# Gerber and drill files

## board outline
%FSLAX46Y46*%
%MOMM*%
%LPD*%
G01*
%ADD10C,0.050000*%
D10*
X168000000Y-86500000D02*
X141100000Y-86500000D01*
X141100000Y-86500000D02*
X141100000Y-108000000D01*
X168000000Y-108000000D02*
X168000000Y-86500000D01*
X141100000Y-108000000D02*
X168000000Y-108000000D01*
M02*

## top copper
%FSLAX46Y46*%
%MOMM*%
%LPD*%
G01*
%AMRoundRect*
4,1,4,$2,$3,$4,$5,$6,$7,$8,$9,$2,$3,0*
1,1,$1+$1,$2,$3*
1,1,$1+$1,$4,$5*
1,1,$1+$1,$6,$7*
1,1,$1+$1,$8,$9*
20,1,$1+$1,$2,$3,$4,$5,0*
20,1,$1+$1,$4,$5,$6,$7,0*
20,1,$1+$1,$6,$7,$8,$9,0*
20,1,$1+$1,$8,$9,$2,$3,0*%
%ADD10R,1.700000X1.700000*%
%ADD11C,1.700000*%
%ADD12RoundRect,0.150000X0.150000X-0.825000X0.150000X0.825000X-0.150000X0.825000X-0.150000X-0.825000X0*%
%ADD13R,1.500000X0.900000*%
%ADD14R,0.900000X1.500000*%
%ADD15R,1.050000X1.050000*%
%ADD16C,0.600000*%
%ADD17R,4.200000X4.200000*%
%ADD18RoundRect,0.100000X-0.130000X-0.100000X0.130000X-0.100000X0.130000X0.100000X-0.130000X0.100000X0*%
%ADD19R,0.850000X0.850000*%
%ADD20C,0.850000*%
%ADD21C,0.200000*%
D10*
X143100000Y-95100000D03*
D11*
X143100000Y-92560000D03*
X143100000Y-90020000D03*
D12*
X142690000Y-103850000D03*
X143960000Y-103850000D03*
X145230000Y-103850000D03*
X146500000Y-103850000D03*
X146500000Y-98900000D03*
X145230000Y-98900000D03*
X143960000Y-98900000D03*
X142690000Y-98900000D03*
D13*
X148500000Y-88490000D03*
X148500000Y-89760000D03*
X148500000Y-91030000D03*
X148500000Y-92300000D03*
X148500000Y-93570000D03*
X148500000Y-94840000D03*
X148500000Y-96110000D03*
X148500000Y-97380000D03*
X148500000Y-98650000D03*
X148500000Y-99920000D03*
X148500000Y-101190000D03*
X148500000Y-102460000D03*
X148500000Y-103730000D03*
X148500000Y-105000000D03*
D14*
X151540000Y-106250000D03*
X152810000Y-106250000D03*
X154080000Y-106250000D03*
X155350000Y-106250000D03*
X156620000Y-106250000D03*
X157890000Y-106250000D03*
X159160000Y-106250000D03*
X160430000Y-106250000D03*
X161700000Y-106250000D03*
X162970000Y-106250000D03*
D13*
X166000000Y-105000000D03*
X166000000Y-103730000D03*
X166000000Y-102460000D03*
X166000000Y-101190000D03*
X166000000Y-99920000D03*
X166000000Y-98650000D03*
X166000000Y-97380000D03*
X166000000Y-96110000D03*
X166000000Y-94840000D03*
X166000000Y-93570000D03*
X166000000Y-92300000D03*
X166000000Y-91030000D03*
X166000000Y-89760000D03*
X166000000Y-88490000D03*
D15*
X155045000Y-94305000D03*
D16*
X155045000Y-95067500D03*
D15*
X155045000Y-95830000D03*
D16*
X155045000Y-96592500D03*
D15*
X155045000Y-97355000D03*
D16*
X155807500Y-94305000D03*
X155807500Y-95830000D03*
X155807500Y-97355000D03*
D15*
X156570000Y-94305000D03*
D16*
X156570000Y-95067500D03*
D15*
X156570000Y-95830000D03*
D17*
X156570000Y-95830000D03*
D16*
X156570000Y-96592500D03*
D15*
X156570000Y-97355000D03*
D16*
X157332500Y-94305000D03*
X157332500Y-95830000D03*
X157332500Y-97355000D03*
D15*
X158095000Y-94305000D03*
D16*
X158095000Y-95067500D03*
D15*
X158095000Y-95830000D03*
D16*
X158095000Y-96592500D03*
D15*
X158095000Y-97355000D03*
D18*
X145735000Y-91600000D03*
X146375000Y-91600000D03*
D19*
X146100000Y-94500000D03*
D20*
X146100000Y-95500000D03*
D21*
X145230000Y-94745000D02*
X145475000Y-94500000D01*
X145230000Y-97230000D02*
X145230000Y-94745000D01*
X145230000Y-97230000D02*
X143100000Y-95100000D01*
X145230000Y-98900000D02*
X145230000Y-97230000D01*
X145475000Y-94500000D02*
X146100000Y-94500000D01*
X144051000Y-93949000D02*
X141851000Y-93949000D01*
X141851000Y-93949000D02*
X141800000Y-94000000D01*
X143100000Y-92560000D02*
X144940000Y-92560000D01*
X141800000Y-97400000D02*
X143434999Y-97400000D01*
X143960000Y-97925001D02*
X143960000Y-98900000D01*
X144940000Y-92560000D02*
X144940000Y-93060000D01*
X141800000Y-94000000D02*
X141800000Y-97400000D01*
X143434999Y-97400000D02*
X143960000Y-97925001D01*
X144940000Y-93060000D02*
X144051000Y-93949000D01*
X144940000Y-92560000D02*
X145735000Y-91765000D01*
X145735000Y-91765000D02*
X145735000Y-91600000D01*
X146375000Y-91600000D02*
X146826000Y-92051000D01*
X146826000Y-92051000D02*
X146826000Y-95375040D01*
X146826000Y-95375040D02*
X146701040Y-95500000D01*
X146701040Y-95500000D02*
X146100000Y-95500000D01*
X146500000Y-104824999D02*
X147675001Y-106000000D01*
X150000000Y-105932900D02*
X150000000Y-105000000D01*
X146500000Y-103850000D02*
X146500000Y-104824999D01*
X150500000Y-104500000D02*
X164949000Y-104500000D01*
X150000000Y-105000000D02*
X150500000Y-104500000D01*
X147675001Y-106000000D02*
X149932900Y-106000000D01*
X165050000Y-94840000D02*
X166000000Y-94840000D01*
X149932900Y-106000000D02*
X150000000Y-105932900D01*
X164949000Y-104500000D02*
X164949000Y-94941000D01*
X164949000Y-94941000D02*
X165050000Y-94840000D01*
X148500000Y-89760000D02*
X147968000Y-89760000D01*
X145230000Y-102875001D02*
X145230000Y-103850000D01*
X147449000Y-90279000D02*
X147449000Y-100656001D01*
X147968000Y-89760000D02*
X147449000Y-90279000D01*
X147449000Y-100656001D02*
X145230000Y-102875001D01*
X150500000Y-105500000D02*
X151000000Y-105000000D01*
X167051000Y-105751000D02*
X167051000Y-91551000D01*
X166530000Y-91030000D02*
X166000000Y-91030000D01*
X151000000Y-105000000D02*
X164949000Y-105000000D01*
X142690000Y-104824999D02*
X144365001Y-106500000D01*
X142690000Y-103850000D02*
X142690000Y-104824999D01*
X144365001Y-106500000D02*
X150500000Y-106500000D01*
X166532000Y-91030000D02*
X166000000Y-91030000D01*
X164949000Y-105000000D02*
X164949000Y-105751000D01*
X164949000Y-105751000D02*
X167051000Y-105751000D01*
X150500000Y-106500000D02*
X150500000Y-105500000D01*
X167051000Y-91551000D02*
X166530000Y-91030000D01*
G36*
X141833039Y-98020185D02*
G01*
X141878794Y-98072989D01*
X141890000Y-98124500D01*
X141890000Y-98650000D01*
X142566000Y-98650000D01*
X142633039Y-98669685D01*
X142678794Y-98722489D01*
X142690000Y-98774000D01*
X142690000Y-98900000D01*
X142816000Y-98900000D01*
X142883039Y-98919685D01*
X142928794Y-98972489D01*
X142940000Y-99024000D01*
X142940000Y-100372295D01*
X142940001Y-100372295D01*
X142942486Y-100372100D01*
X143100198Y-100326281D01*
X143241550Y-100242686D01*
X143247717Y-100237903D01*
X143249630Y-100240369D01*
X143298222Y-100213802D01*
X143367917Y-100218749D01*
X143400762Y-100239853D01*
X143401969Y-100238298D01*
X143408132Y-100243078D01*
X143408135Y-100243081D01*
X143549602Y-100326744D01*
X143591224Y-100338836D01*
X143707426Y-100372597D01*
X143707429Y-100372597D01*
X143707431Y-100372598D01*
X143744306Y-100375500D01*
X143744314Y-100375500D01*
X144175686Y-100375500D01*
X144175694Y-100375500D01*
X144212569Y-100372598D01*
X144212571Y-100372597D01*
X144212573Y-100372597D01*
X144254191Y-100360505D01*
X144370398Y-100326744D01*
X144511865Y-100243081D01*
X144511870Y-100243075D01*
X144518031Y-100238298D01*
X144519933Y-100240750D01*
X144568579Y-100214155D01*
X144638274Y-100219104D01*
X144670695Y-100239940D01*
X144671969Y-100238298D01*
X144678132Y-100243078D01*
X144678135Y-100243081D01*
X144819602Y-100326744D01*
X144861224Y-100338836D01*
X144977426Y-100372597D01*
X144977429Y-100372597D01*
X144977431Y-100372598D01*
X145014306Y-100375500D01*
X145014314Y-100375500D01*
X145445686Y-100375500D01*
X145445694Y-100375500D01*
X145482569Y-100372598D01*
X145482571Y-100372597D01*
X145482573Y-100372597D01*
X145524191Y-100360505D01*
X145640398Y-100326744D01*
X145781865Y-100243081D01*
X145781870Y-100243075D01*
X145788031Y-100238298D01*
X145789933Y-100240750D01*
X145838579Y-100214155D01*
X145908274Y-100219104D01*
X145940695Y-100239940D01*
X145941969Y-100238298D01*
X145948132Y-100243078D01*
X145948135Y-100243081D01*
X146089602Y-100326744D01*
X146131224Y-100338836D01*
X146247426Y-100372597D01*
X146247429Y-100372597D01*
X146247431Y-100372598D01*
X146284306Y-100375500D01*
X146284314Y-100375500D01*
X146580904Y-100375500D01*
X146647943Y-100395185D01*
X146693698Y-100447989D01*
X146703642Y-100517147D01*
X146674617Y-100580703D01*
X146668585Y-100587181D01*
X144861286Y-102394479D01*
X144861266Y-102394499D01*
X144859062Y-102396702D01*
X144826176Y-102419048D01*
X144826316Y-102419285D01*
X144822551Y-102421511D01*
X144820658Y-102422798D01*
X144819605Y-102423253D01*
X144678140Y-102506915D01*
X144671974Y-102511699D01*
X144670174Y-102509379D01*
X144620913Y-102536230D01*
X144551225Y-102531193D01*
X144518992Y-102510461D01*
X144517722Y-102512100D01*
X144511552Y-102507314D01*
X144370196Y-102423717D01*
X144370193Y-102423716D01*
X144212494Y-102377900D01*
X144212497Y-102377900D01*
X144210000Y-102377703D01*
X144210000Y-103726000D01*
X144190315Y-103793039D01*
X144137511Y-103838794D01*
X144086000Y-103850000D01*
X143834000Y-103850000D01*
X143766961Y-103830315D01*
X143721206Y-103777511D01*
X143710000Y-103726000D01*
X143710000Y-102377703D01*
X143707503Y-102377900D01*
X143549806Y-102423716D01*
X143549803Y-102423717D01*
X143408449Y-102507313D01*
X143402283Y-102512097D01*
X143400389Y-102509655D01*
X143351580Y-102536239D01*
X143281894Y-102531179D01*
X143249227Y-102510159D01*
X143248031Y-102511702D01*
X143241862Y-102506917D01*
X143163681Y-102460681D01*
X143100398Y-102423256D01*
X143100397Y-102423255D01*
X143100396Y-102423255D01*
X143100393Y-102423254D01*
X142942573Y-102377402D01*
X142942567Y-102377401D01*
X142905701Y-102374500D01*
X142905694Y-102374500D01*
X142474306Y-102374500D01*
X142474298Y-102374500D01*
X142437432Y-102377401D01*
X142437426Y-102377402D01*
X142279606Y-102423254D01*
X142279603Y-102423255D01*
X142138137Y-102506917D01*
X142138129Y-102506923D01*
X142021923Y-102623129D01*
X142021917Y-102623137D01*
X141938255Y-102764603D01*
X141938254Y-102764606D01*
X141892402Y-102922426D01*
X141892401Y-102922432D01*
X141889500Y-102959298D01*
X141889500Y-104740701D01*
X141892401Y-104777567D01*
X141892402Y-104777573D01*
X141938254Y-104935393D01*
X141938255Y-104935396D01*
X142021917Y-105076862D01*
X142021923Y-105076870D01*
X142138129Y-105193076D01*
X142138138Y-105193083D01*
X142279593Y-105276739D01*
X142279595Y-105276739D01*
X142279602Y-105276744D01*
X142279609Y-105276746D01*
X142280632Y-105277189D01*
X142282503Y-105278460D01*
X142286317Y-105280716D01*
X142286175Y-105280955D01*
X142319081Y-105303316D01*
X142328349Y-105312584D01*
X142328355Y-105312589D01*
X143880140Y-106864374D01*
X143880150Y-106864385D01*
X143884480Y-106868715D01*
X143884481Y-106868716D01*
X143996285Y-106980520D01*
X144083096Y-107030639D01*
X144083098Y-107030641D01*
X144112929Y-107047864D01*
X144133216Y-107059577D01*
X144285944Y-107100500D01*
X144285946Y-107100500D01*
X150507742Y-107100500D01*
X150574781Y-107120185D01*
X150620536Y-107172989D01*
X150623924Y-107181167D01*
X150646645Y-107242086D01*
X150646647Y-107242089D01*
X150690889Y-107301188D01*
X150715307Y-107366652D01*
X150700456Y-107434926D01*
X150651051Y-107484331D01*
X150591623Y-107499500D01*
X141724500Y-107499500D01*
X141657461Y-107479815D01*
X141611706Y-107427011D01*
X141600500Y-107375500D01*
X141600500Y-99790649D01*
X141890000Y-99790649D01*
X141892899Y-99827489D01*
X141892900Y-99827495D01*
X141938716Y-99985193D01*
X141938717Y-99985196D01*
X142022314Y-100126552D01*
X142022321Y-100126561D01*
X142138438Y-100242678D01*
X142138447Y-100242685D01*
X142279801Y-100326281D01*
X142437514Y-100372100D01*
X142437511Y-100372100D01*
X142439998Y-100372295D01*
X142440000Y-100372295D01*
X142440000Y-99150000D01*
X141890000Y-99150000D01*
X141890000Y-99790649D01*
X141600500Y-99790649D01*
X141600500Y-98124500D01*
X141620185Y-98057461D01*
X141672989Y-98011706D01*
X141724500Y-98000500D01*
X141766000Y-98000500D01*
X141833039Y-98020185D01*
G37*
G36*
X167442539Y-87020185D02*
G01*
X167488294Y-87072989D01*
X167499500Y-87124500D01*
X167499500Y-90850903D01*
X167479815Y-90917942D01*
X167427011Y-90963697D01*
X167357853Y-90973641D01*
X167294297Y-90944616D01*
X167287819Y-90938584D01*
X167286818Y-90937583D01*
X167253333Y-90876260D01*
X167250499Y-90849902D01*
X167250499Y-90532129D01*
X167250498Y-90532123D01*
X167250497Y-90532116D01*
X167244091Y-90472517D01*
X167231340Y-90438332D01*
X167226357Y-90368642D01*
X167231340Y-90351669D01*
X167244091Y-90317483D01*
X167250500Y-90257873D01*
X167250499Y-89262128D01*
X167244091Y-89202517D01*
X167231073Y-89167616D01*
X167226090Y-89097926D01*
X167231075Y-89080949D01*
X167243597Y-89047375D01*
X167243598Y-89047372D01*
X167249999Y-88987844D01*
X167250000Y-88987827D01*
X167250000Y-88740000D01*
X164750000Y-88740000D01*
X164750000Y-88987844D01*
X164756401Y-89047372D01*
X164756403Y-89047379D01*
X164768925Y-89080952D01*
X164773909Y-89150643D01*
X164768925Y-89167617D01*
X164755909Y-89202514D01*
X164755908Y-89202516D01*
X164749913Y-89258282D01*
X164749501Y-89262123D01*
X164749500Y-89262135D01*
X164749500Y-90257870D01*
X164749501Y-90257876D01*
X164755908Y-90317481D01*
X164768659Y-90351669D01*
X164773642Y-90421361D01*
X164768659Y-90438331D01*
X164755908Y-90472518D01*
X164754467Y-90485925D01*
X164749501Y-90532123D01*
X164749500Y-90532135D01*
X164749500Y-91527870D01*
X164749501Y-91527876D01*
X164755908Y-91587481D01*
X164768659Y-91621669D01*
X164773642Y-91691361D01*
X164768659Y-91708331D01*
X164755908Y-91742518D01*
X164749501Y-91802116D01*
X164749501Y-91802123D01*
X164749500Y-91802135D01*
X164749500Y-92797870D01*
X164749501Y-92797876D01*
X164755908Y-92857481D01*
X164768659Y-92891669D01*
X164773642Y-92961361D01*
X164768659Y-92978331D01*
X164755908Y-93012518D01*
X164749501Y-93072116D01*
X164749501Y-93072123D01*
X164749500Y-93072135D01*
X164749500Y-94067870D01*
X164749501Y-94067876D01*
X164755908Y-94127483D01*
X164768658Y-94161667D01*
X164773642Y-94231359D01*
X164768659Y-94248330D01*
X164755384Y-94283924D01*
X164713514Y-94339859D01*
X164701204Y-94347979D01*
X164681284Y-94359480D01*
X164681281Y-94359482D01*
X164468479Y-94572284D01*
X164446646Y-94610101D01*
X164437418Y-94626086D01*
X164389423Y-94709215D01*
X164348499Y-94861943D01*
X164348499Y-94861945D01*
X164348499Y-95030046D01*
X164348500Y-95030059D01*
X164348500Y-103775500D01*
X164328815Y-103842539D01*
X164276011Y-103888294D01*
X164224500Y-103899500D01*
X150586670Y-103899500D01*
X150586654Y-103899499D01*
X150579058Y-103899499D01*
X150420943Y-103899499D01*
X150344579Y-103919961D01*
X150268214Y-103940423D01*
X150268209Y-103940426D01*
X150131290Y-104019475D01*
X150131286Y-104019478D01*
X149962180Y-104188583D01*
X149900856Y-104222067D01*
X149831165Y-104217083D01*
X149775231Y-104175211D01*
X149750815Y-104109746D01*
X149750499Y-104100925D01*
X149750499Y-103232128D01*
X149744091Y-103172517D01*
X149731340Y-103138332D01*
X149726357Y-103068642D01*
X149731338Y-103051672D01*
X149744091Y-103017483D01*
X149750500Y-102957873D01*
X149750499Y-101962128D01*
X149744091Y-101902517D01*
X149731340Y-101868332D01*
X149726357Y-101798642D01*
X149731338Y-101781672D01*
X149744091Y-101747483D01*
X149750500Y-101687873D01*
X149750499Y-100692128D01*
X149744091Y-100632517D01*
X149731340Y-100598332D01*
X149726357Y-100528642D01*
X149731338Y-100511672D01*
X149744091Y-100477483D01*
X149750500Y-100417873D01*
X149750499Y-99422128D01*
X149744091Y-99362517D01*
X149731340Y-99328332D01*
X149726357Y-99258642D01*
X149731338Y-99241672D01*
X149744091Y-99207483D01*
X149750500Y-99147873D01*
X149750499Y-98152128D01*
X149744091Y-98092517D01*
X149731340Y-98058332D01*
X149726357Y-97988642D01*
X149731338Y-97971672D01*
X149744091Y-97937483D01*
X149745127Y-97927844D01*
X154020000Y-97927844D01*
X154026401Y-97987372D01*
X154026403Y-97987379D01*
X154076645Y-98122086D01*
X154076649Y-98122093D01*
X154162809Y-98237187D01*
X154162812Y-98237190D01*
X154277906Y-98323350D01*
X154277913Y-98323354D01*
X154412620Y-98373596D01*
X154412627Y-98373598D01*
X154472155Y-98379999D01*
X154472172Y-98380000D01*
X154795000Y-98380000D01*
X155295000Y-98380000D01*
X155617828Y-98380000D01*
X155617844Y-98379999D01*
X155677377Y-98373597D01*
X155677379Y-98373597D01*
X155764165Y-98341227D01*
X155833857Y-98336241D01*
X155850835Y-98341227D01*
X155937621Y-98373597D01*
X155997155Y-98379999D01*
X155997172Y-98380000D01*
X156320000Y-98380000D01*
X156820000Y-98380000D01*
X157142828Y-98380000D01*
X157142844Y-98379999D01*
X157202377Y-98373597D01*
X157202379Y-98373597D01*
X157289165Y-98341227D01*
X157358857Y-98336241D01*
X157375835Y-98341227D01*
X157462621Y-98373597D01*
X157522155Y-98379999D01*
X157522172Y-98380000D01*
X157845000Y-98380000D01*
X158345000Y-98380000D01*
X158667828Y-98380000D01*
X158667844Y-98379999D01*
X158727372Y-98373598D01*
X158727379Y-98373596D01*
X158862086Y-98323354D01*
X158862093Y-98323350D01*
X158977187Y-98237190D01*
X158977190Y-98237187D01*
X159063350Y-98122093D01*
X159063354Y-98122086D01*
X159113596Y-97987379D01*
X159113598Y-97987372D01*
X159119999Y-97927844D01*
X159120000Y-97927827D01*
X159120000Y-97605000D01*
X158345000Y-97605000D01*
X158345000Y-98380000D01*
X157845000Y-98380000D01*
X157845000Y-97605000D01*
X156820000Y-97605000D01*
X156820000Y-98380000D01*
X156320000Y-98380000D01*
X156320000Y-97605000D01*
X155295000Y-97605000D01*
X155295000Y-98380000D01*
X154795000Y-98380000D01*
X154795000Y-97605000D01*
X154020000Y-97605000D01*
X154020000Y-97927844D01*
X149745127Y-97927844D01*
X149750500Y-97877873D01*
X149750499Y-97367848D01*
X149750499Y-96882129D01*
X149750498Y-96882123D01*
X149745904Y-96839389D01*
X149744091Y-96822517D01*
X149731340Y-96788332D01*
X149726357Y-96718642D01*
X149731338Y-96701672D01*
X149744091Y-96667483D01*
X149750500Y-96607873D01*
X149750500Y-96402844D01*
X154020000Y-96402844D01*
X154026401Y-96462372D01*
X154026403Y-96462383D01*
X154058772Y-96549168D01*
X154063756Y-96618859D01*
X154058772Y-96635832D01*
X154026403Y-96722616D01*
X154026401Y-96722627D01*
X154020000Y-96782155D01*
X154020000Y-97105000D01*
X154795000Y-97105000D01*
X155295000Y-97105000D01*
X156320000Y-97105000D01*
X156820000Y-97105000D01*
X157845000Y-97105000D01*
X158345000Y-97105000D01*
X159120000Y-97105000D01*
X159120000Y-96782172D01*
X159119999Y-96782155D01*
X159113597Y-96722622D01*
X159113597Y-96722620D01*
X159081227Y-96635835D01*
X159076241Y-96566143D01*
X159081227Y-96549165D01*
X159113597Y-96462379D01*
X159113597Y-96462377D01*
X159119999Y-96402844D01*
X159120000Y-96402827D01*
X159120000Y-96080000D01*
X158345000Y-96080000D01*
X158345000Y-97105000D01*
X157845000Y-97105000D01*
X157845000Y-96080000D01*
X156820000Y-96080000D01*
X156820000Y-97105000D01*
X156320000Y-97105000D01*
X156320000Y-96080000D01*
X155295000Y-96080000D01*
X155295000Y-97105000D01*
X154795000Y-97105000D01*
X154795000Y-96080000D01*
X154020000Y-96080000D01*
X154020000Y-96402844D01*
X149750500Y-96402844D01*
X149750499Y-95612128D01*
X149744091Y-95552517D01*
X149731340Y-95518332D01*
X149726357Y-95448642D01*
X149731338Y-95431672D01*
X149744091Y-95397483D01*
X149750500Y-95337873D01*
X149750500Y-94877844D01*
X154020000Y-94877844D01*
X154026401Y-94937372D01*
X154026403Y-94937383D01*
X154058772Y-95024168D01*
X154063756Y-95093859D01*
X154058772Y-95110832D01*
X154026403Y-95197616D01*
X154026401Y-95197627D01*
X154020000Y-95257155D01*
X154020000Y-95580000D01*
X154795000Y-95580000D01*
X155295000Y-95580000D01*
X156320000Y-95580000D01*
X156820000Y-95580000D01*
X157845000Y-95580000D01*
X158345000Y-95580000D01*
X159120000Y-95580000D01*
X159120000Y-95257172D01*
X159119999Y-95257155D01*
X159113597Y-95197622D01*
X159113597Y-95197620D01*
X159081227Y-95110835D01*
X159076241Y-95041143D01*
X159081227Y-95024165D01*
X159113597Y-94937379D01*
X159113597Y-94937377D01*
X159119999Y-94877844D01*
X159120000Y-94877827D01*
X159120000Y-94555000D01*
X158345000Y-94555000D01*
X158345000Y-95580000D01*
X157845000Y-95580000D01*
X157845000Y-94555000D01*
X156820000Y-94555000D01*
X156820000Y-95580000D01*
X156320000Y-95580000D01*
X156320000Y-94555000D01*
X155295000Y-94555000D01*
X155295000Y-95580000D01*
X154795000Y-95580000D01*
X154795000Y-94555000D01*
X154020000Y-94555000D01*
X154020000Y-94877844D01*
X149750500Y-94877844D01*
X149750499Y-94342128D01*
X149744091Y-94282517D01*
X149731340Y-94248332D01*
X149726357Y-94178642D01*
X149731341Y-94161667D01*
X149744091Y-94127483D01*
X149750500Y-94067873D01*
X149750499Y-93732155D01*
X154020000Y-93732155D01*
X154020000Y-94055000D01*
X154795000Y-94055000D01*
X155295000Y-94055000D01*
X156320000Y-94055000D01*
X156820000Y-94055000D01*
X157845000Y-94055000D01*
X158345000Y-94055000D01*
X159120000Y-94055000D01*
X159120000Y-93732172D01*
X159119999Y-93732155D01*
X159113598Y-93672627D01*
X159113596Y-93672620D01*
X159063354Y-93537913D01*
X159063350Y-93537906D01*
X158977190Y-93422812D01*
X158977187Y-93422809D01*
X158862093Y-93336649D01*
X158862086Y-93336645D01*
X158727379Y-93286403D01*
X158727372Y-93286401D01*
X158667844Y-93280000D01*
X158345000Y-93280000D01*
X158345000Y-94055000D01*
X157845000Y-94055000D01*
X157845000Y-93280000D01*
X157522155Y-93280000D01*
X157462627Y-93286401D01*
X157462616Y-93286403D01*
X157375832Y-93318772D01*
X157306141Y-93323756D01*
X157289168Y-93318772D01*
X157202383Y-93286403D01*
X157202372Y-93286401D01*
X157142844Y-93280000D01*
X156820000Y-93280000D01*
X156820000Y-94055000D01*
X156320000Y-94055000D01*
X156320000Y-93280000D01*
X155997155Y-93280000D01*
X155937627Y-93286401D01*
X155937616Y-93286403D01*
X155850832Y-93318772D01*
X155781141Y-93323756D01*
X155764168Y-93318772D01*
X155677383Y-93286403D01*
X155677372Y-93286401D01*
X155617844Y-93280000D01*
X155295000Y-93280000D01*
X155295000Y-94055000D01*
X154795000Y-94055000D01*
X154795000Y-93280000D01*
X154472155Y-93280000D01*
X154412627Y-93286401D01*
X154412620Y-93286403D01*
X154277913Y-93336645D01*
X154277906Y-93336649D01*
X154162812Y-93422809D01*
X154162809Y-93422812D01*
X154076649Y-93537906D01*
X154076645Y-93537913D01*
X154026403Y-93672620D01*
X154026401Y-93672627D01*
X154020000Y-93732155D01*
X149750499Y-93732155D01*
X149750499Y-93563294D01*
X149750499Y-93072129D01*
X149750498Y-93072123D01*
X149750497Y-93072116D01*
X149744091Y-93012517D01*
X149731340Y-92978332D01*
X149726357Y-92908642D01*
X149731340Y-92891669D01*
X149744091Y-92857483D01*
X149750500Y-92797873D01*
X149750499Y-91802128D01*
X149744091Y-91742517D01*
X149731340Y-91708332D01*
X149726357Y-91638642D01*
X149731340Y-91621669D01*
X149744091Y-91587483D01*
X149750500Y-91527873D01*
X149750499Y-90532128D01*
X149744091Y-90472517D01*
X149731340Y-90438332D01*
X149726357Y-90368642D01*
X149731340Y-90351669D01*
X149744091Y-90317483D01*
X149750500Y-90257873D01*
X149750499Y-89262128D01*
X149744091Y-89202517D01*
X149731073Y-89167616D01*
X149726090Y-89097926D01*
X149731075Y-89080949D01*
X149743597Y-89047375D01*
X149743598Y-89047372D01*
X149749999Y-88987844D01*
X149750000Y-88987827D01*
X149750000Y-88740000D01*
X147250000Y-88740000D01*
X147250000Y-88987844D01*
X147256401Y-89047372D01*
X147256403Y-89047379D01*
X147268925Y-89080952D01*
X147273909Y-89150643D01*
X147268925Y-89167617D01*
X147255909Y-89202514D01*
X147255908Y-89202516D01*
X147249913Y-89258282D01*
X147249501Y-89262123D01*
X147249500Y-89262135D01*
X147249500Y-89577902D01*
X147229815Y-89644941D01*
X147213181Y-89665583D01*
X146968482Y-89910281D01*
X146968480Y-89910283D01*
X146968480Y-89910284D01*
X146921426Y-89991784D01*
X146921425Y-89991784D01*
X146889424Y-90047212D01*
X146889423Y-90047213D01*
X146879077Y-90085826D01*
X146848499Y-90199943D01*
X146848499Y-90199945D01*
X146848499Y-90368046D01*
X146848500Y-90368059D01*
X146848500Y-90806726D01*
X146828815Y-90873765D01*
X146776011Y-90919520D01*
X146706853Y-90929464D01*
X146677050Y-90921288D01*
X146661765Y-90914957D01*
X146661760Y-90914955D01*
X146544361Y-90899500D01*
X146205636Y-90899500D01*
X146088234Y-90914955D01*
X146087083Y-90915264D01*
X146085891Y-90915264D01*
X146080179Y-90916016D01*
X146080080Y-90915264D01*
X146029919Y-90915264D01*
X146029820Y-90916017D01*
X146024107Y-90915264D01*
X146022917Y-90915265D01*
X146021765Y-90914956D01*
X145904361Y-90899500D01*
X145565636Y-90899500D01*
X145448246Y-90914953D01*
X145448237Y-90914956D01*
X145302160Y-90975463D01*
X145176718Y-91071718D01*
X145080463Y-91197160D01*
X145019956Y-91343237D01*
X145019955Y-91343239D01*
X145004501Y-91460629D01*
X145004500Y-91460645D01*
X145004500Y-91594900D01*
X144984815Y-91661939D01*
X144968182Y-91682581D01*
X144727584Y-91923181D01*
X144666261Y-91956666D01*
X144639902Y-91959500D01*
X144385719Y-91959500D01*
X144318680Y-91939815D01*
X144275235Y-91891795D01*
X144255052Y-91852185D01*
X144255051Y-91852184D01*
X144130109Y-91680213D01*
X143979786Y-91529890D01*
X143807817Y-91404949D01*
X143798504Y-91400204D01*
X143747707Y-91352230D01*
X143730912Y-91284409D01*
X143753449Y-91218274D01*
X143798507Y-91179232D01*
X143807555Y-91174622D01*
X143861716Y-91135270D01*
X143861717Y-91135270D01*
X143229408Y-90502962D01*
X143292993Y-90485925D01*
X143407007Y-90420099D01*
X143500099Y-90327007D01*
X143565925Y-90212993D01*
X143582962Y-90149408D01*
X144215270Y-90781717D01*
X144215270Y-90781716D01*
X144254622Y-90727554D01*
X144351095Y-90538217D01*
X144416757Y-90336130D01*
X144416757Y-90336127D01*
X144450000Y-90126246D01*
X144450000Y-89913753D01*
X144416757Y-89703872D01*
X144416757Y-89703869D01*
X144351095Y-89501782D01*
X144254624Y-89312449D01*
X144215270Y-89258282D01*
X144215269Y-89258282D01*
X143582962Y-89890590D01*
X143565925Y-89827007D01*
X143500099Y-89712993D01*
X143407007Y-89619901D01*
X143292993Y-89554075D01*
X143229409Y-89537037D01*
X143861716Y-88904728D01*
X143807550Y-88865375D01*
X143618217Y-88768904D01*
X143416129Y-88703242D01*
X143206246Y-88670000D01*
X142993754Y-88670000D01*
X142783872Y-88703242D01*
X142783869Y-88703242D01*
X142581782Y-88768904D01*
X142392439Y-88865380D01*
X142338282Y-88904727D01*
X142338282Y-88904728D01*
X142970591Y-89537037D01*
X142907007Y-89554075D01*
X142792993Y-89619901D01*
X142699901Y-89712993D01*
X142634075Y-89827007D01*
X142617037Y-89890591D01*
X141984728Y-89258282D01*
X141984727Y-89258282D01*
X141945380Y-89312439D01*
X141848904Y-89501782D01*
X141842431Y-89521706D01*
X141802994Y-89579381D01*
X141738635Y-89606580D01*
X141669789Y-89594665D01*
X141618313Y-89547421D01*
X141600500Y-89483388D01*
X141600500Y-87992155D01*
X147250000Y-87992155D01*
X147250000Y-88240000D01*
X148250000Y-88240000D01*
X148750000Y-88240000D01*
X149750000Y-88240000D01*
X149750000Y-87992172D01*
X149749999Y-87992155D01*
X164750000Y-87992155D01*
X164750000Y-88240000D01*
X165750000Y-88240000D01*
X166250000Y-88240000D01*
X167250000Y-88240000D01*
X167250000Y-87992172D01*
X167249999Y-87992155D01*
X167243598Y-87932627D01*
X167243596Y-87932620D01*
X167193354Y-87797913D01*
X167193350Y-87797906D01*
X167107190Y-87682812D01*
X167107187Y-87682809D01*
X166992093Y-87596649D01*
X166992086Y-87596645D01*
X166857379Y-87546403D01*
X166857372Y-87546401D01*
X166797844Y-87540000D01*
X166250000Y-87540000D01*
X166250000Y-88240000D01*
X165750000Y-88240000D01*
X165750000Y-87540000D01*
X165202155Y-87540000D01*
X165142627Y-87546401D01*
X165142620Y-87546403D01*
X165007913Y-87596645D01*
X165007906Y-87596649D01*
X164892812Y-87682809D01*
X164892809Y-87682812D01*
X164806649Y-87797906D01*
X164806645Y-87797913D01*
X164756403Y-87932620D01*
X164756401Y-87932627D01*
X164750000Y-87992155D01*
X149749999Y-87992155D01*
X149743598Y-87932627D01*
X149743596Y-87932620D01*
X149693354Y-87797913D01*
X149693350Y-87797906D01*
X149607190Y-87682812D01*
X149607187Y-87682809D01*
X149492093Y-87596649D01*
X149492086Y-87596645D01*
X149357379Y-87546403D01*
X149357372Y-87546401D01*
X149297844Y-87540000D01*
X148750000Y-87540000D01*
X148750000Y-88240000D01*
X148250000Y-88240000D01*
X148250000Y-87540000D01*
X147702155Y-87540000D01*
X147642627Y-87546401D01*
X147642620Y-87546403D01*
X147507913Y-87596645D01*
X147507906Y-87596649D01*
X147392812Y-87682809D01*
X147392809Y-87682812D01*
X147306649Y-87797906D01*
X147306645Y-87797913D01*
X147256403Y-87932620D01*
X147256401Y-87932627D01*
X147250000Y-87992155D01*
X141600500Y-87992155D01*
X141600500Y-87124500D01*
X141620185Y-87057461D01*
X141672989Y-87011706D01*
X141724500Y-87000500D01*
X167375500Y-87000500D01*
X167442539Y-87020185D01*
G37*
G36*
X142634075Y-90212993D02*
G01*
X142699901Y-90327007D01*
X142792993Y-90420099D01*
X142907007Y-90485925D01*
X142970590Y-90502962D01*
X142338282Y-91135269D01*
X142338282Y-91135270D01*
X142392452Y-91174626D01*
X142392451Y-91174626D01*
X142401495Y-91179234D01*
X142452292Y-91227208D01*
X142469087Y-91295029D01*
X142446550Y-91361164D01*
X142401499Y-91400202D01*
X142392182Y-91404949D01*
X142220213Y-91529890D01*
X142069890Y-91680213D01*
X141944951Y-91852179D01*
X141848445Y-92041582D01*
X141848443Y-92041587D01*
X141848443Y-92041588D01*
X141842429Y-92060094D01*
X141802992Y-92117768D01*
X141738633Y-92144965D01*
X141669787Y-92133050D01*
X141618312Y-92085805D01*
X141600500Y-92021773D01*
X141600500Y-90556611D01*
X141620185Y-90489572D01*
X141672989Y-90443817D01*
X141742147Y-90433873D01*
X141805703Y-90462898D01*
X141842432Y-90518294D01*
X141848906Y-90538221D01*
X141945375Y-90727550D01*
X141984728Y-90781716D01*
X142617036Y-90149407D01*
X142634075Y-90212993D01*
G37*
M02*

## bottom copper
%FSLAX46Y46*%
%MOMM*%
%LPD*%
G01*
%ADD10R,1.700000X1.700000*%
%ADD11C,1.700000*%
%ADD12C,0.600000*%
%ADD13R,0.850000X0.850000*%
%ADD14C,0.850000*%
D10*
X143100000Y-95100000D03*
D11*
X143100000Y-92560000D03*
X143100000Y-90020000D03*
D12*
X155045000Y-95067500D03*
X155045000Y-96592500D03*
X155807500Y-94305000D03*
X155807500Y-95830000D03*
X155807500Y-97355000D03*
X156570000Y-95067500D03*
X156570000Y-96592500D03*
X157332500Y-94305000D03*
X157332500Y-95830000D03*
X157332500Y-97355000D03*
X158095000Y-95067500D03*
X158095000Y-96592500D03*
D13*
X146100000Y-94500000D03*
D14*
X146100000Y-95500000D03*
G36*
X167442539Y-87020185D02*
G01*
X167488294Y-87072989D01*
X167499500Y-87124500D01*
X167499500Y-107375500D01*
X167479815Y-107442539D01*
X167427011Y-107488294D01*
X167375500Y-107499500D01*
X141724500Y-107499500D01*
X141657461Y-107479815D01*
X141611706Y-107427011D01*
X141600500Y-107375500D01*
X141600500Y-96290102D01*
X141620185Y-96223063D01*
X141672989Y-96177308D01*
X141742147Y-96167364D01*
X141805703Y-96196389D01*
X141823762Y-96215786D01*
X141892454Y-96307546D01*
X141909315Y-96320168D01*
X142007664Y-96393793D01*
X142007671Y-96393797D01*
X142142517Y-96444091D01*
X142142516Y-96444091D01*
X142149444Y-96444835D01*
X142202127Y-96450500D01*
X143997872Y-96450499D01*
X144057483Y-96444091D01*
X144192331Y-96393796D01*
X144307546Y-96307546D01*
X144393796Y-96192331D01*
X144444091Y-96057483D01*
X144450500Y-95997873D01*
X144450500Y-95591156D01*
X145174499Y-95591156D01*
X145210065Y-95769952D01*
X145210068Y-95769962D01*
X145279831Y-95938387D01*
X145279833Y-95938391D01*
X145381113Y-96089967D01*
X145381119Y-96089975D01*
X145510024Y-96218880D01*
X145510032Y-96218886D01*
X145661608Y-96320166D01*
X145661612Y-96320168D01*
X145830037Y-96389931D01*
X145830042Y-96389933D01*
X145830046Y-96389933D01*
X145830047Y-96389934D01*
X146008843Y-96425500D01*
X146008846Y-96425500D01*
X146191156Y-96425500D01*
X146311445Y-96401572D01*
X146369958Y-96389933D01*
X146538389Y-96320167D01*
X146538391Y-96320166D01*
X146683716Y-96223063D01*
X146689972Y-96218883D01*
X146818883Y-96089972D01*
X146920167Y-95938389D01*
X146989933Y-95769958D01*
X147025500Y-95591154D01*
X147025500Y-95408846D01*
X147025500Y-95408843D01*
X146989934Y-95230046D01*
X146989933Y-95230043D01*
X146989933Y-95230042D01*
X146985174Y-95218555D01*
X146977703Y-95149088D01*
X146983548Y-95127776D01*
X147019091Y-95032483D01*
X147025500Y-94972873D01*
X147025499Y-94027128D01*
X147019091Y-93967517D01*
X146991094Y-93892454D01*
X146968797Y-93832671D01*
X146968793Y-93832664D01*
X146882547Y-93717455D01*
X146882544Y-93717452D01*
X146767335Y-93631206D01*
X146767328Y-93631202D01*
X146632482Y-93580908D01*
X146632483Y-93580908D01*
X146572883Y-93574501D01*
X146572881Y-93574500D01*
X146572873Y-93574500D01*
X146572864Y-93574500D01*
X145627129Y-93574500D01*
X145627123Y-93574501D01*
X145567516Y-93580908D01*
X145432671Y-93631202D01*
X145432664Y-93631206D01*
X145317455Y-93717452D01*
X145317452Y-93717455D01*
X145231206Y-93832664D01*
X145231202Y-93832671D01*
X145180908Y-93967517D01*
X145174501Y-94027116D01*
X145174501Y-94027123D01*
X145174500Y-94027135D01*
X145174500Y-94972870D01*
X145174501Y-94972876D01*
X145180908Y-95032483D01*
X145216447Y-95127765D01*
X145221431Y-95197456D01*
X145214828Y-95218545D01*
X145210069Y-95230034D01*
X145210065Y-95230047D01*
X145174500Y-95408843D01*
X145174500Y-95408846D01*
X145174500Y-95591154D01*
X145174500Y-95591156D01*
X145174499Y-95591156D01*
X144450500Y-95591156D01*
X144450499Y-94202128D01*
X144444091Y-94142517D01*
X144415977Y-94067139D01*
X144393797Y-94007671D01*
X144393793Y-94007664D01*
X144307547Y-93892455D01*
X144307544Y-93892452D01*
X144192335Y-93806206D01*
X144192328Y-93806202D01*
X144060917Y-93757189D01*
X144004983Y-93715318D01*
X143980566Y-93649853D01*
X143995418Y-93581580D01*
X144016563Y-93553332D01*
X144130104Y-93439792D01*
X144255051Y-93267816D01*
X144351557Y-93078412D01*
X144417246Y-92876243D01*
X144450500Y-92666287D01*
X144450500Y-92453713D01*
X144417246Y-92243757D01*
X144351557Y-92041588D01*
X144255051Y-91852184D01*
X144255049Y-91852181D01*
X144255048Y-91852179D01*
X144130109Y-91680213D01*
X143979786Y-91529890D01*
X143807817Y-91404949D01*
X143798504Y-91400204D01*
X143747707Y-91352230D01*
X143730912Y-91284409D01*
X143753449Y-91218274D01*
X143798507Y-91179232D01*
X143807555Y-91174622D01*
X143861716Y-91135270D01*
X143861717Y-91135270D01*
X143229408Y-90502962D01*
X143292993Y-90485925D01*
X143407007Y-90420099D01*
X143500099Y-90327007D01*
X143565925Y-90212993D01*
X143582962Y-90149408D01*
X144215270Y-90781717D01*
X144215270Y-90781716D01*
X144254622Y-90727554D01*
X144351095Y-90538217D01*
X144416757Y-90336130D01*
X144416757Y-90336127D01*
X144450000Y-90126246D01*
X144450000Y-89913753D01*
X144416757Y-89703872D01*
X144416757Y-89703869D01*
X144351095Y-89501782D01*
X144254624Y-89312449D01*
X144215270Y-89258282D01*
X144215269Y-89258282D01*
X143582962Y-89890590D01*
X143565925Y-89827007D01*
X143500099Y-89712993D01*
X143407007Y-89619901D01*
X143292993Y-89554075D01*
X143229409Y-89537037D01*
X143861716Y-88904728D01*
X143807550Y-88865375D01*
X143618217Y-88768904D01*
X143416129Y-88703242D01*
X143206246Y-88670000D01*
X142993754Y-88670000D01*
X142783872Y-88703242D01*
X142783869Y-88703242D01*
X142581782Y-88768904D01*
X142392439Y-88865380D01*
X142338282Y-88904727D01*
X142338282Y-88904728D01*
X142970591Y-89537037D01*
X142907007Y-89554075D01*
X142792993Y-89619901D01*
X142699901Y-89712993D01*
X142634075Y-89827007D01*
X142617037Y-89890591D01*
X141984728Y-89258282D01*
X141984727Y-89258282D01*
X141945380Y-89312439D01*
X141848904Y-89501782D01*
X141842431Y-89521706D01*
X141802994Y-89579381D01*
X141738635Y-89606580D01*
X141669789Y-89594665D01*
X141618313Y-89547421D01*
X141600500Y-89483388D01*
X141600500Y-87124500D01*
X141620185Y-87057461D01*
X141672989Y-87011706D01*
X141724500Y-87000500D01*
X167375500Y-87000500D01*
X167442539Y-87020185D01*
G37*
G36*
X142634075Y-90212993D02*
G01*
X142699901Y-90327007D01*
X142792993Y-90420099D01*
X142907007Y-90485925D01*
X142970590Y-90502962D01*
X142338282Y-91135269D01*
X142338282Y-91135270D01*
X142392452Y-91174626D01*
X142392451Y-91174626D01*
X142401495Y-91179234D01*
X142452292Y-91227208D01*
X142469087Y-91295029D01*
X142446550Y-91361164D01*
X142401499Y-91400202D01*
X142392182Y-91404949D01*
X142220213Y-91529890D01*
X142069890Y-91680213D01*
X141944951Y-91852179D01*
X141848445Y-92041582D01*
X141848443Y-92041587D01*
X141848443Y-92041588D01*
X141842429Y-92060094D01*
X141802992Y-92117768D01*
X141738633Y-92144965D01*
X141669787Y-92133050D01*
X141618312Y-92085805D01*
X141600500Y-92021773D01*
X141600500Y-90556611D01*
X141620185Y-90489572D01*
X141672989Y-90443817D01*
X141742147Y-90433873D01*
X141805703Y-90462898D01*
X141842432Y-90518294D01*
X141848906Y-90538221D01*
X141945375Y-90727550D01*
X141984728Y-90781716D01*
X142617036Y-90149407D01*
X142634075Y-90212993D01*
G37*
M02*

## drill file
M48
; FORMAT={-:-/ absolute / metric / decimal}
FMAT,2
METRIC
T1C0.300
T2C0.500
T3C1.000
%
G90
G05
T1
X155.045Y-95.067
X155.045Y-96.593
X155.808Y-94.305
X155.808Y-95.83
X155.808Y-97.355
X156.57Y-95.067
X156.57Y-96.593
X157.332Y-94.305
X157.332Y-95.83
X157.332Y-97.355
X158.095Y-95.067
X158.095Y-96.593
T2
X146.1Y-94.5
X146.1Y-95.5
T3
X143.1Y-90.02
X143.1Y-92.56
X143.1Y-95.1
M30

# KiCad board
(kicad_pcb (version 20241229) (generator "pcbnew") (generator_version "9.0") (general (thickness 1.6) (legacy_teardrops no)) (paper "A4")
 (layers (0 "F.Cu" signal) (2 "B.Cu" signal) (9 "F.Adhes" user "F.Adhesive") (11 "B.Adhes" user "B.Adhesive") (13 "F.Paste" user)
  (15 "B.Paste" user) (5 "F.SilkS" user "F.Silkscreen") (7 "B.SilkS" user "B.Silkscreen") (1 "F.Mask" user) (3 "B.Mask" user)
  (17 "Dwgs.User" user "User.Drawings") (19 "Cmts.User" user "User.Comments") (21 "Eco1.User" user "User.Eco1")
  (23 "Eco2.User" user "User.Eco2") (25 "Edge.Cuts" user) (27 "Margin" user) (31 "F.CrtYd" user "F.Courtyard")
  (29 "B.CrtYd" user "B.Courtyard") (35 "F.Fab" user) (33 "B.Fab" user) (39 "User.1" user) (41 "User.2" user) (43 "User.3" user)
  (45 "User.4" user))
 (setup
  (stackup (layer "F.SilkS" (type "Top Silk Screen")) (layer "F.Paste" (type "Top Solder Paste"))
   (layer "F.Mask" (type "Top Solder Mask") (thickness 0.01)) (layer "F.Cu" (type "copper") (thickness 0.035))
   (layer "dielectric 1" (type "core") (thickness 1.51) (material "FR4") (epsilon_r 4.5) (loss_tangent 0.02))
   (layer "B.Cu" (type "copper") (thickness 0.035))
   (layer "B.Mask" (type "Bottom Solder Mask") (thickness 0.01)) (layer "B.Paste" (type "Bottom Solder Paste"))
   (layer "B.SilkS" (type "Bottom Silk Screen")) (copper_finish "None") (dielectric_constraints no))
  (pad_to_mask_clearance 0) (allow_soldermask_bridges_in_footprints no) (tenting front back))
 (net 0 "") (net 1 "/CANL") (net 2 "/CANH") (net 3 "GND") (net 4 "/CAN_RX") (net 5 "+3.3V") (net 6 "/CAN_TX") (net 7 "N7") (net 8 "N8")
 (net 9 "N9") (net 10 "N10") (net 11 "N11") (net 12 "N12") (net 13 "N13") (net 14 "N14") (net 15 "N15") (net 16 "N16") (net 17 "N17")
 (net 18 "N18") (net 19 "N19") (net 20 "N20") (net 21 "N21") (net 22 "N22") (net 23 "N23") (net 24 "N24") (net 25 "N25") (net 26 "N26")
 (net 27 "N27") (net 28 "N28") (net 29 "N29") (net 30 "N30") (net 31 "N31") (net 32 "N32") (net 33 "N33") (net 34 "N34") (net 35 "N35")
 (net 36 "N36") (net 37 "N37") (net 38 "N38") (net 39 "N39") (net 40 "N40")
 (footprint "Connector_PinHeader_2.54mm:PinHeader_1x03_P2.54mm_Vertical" (layer "F.Cu") (at 143.1 95.1 180)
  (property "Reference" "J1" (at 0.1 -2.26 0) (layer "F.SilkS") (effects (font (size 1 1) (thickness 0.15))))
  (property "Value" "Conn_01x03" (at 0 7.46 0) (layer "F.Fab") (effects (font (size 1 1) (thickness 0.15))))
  (pad "1" thru_hole rect (at 0 0 180) (size 1.7 1.7) (drill 1) (layers "*.Cu" "*.Mask") (remove_unused_layers no) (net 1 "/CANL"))
  (pad "2" thru_hole circle (at 0 2.54 180) (size 1.7 1.7) (drill 1) (layers "*.Cu" "*.Mask") (remove_unused_layers no) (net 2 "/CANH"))
  (pad "3" thru_hole circle (at 0 5.08 180) (size 1.7 1.7) (drill 1) (layers "*.Cu" "*.Mask") (remove_unused_layers no) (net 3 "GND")))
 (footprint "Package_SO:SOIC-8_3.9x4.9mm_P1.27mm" (layer "F.Cu") (at 144.595 101.375 90)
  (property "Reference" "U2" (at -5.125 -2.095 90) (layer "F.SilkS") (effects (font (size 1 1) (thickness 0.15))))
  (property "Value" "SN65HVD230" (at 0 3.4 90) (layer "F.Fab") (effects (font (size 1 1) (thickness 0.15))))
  (pad "1" smd roundrect (at -2.475 -1.905 90) (size 1.95 0.6) (layers "F.Cu" "F.Mask" "F.Paste") (roundrect_rratio 0.25) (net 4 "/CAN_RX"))
  (pad "2" smd roundrect (at -2.475 -0.635 90) (size 1.95 0.6) (layers "F.Cu" "F.Mask" "F.Paste") (roundrect_rratio 0.25) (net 3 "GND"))
  (pad "3" smd roundrect (at -2.475 0.635 90) (size 1.95 0.6) (layers "F.Cu" "F.Mask" "F.Paste") (roundrect_rratio 0.25) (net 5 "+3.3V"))
  (pad "4" smd roundrect (at -2.475 1.905 90) (size 1.95 0.6) (layers "F.Cu" "F.Mask" "F.Paste") (roundrect_rratio 0.25) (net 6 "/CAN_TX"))
  (pad "5" smd roundrect (at 2.475 1.905 90) (size 1.95 0.6) (layers "F.Cu" "F.Mask" "F.Paste") (roundrect_rratio 0.25) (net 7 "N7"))
  (pad "6" smd roundrect (at 2.475 0.635 90) (size 1.95 0.6) (layers "F.Cu" "F.Mask" "F.Paste") (roundrect_rratio 0.25) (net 1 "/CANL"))
  (pad "7" smd roundrect (at 2.475 -0.635 90) (size 1.95 0.6) (layers "F.Cu" "F.Mask" "F.Paste") (roundrect_rratio 0.25) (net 2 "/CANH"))
  (pad "8" smd roundrect (at 2.475 -1.905 90) (size 1.95 0.6) (layers "F.Cu" "F.Mask" "F.Paste") (roundrect_rratio 0.25) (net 3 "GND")))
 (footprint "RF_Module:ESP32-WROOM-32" (layer "F.Cu") (at 157.25 96.74)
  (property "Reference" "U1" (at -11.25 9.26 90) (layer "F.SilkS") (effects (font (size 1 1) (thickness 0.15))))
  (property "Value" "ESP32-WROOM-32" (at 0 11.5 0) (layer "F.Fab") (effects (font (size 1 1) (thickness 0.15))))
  (pad "1" smd rect (at -8.75 -8.25) (size 1.5 0.9) (layers "F.Cu" "F.Mask" "F.Paste") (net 3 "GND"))
  (pad "2" smd rect (at -8.75 -6.98) (size 1.5 0.9) (layers "F.Cu" "F.Mask" "F.Paste") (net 5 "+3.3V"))
  (pad "3" smd rect (at -8.75 -5.71) (size 1.5 0.9) (layers "F.Cu" "F.Mask" "F.Paste") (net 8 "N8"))
  (pad "4" smd rect (at -8.75 -4.44) (size 1.5 0.9) (layers "F.Cu" "F.Mask" "F.Paste") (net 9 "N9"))
  (pad "5" smd rect (at -8.75 -3.17) (size 1.5 0.9) (layers "F.Cu" "F.Mask" "F.Paste") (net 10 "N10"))
  (pad "6" smd rect (at -8.75 -1.9) (size 1.5 0.9) (layers "F.Cu" "F.Mask" "F.Paste") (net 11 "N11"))
  (pad "7" smd rect (at -8.75 -0.63) (size 1.5 0.9) (layers "F.Cu" "F.Mask" "F.Paste") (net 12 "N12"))
  (pad "8" smd rect (at -8.75 0.64) (size 1.5 0.9) (layers "F.Cu" "F.Mask" "F.Paste") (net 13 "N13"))
  (pad "9" smd rect (at -8.75 1.91) (size 1.5 0.9) (layers "F.Cu" "F.Mask" "F.Paste") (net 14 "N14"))
  (pad "10" smd rect (at -8.75 3.18) (size 1.5 0.9) (layers "F.Cu" "F.Mask" "F.Paste") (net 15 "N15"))
  (pad "11" smd rect (at -8.75 4.45) (size 1.5 0.9) (layers "F.Cu" "F.Mask" "F.Paste") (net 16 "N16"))
  (pad "12" smd rect (at -8.75 5.72) (size 1.5 0.9) (layers "F.Cu" "F.Mask" "F.Paste") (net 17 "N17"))
  (pad "13" smd rect (at -8.75 6.99) (size 1.5 0.9) (layers "F.Cu" "F.Mask" "F.Paste") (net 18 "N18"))
  (pad "14" smd rect (at -8.75 8.26) (size 1.5 0.9) (layers "F.Cu" "F.Mask" "F.Paste") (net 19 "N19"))
  (pad "15" smd rect (at -5.71 9.51 90) (size 1.5 0.9) (layers "F.Cu" "F.Mask" "F.Paste") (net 3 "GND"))
  (pad "16" smd rect (at -4.44 9.51 90) (size 1.5 0.9) (layers "F.Cu" "F.Mask" "F.Paste") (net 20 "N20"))
  (pad "17" smd rect (at -3.17 9.51 90) (size 1.5 0.9) (layers "F.Cu" "F.Mask" "F.Paste") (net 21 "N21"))
  (pad "18" smd rect (at -1.9 9.51 90) (size 1.5 0.9) (layers "F.Cu" "F.Mask" "F.Paste") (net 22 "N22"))
  (pad "19" smd rect (at -0.63 9.51 90) (size 1.5 0.9) (layers "F.Cu" "F.Mask" "F.Paste") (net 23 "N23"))
  (pad "20" smd rect (at 0.64 9.51 90) (size 1.5 0.9) (layers "F.Cu" "F.Mask" "F.Paste") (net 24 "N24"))
  (pad "21" smd rect (at 1.91 9.51 90) (size 1.5 0.9) (layers "F.Cu" "F.Mask" "F.Paste") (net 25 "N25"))
  (pad "22" smd rect (at 3.18 9.51 90) (size 1.5 0.9) (layers "F.Cu" "F.Mask" "F.Paste") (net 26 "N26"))
  (pad "23" smd rect (at 4.45 9.51 90) (size 1.5 0.9) (layers "F.Cu" "F.Mask" "F.Paste") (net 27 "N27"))
  (pad "24" smd rect (at 5.72 9.51 90) (size 1.5 0.9) (layers "F.Cu" "F.Mask" "F.Paste") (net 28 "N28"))
  (pad "25" smd rect (at 8.75 8.26) (size 1.5 0.9) (layers "F.Cu" "F.Mask" "F.Paste") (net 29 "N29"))
  (pad "26" smd rect (at 8.75 6.99) (size 1.5 0.9) (layers "F.Cu" "F.Mask" "F.Paste") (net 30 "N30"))
  (pad "27" smd rect (at 8.75 5.72) (size 1.5 0.9) (layers "F.Cu" "F.Mask" "F.Paste") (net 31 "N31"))
  (pad "28" smd rect (at 8.75 4.45) (size 1.5 0.9) (layers "F.Cu" "F.Mask" "F.Paste") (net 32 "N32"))
  (pad "29" smd rect (at 8.75 3.18) (size 1.5 0.9) (layers "F.Cu" "F.Mask" "F.Paste") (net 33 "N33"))
  (pad "30" smd rect (at 8.75 1.91) (size 1.5 0.9) (layers "F.Cu" "F.Mask" "F.Paste") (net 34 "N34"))
  (pad "31" smd rect (at 8.75 0.64) (size 1.5 0.9) (layers "F.Cu" "F.Mask" "F.Paste") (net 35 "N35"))
  (pad "32" smd rect (at 8.75 -0.63) (size 1.5 0.9) (layers "F.Cu" "F.Mask" "F.Paste") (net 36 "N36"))
  (pad "33" smd rect (at 8.75 -1.9) (size 1.5 0.9) (layers "F.Cu" "F.Mask" "F.Paste") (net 6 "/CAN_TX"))
  (pad "34" smd rect (at 8.75 -3.17) (size 1.5 0.9) (layers "F.Cu" "F.Mask" "F.Paste") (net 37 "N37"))
  (pad "35" smd rect (at 8.75 -4.44) (size 1.5 0.9) (layers "F.Cu" "F.Mask" "F.Paste") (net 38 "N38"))
  (pad "36" smd rect (at 8.75 -5.71) (size 1.5 0.9) (layers "F.Cu" "F.Mask" "F.Paste") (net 4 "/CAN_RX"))
  (pad "37" smd rect (at 8.75 -6.98) (size 1.5 0.9) (layers "F.Cu" "F.Mask" "F.Paste") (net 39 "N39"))
  (pad "38" smd rect (at 8.75 -8.25) (size 1.5 0.9) (layers "F.Cu" "F.Mask" "F.Paste") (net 3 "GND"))
  (pad "39" smd rect (at -2.205 -2.435) (size 1.05 1.05) (layers "F.Cu" "F.Paste") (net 3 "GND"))
  (pad "39" thru_hole circle (at -2.205 -1.6725) (size 0.6 0.6) (drill 0.3) (layers "*.Cu" "F.Mask") (remove_unused_layers no) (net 3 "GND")
   (zone_connect 2))
  (pad "39" smd rect (at -2.205 -0.91) (size 1.05 1.05) (layers "F.Cu" "F.Paste") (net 3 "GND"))
  (pad "39" thru_hole circle (at -2.205 -0.1475) (size 0.6 0.6) (drill 0.3) (layers "*.Cu" "F.Mask") (remove_unused_layers no) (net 3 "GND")
   (zone_connect 2))
  (pad "39" smd rect (at -2.205 0.615) (size 1.05 1.05) (layers "F.Cu" "F.Paste") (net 3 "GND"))
  (pad "39" thru_hole circle (at -1.4425 -2.435) (size 0.6 0.6) (drill 0.3) (layers "*.Cu" "F.Mask") (remove_unused_layers no) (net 3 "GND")
   (zone_connect 2))
  (pad "39" thru_hole circle (at -1.4425 -0.91) (size 0.6 0.6) (drill 0.3) (layers "*.Cu" "F.Mask") (remove_unused_layers no) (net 3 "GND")
   (zone_connect 2))
  (pad "39" thru_hole circle (at -1.4425 0.615) (size 0.6 0.6) (drill 0.3) (layers "*.Cu" "F.Mask") (remove_unused_layers no) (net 3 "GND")
   (zone_connect 2))
  (pad "39" smd rect (at -0.68 -2.435) (size 1.05 1.05) (layers "F.Cu" "F.Paste") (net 3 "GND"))
  (pad "39" thru_hole circle (at -0.68 -1.6725) (size 0.6 0.6) (drill 0.3) (layers "*.Cu" "F.Mask") (remove_unused_layers no) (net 3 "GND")
   (zone_connect 2))
  (pad "39" smd rect (at -0.68 -0.91) (size 1.05 1.05) (layers "F.Cu" "F.Paste") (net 3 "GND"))
  (pad "39" smd rect (at -0.68 -0.91) (size 4.2 4.2) (layers "F.Cu" "F.Mask") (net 3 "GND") (zone_connect 2))
  (pad "39" thru_hole circle (at -0.68 -0.1475) (size 0.6 0.6) (drill 0.3) (layers "*.Cu" "F.Mask") (remove_unused_layers no) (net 3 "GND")
   (zone_connect 2))
  (pad "39" smd rect (at -0.68 0.615) (size 1.05 1.05) (layers "F.Cu" "F.Paste") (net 3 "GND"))
  (pad "39" thru_hole circle (at 0.0825 -2.435) (size 0.6 0.6) (drill 0.3) (layers "*.Cu" "F.Mask") (remove_unused_layers no) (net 3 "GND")
   (zone_connect 2))
  (pad "39" thru_hole circle (at 0.0825 -0.91) (size 0.6 0.6) (drill 0.3) (layers "*.Cu" "F.Mask") (remove_unused_layers no) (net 3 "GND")
   (zone_connect 2))
  (pad "39" thru_hole circle (at 0.0825 0.615) (size 0.6 0.6) (drill 0.3) (layers "*.Cu" "F.Mask") (remove_unused_layers no) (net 3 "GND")
   (zone_connect 2))
  (pad "39" smd rect (at 0.845 -2.435) (size 1.05 1.05) (layers "F.Cu" "F.Paste") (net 3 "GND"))
  (pad "39" thru_hole circle (at 0.845 -1.6725) (size 0.6 0.6) (drill 0.3) (layers "*.Cu" "F.Mask") (remove_unused_layers no) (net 3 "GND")
   (zone_connect 2))
  (pad "39" smd rect (at 0.845 -0.91) (size 1.05 1.05) (layers "F.Cu" "F.Paste") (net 3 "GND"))
  (pad "39" thru_hole circle (at 0.845 -0.1475) (size 0.6 0.6) (drill 0.3) (layers "*.Cu" "F.Mask") (remove_unused_layers no) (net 3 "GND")
   (zone_connect 2))
  (pad "39" smd rect (at 0.845 0.615) (size 1.05 1.05) (layers "F.Cu" "F.Paste") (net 3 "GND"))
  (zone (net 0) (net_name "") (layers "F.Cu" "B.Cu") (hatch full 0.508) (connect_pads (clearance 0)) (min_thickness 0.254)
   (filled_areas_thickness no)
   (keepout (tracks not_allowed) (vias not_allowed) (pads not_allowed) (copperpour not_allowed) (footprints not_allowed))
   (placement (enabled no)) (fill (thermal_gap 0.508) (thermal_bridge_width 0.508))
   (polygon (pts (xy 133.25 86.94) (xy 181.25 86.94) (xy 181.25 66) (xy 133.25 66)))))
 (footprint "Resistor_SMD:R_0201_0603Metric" (layer "F.Cu") (at 146.055 91.6)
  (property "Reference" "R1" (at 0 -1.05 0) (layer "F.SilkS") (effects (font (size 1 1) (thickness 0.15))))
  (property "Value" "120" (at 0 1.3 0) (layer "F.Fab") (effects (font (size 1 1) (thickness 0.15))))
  (pad "" smd roundrect (at -0.345 0) (size 0.318 0.36) (layers "F.Paste") (roundrect_rratio 0.25))
  (pad "" smd roundrect (at 0.345 0) (size 0.318 0.36) (layers "F.Paste") (roundrect_rratio 0.25))
  (pad "1" smd roundrect (at -0.32 0) (size 0.46 0.4) (layers "F.Cu" "F.Mask") (roundrect_rratio 0.25) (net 2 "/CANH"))
  (pad "2" smd roundrect (at 0.32 0) (size 0.46 0.4) (layers "F.Cu" "F.Mask") (roundrect_rratio 0.25) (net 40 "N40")))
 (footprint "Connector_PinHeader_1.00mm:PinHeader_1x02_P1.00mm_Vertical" (layer "F.Cu") (at 146.1 94.5)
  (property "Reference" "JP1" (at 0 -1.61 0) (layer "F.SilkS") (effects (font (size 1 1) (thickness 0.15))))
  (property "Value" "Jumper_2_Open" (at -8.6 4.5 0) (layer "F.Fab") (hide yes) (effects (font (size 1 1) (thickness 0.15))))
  (pad "1" thru_hole rect (at 0 0) (size 0.85 0.85) (drill 0.5) (layers "*.Cu" "*.Mask") (remove_unused_layers no) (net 1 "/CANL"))
  (pad "2" thru_hole circle (at 0 1) (size 0.85 0.85) (drill 0.5) (layers "*.Cu" "*.Mask") (remove_unused_layers no) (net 40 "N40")))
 (gr_line (start 168 86.5) (end 141.1 86.5) (stroke (width 0.05) (type default)) (layer "Edge.Cuts"))
 (gr_line (start 141.1 86.5) (end 141.1 108) (stroke (width 0.05) (type default)) (layer "Edge.Cuts"))
 (gr_line (start 168 108) (end 168 86.5) (stroke (width 0.05) (type default)) (layer "Edge.Cuts"))
 (gr_line (start 141.1 108) (end 168 108) (stroke (width 0.05) (type default)) (layer "Edge.Cuts"))
 (segment (start 145.23 94.745) (end 145.475 94.5) (width 0.2) (layer "F.Cu") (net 1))
 (segment (start 145.23 97.23) (end 145.23 94.745) (width 0.2) (layer "F.Cu") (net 1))
 (segment (start 145.23 97.23) (end 143.1 95.1) (width 0.2) (layer "F.Cu") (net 1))
 (segment (start 145.23 98.9) (end 145.23 97.23) (width 0.2) (layer "F.Cu") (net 1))
 (segment (start 145.475 94.5) (end 146.1 94.5) (width 0.2) (layer "F.Cu") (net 1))
 (segment (start 144.051 93.949) (end 141.851 93.949) (width 0.2) (layer "F.Cu") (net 2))
 (segment (start 141.851 93.949) (end 141.8 94) (width 0.2) (layer "F.Cu") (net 2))
 (segment (start 143.1 92.56) (end 144.94 92.56) (width 0.2) (layer "F.Cu") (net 2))
 (segment (start 141.8 97.4) (end 143.434999 97.4) (width 0.2) (layer "F.Cu") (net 2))
 (segment (start 143.96 97.925001) (end 143.96 98.9) (width 0.2) (layer "F.Cu") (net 2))
 (segment (start 144.94 92.56) (end 144.94 93.06) (width 0.2) (layer "F.Cu") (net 2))
 (segment (start 141.8 94) (end 141.8 97.4) (width 0.2) (layer "F.Cu") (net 2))
 (segment (start 143.434999 97.4) (end 143.96 97.925001) (width 0.2) (layer "F.Cu") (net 2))
 (segment (start 144.94 93.06) (end 144.051 93.949) (width 0.2) (layer "F.Cu") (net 2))
 (segment (start 144.94 92.56) (end 145.735 91.765) (width 0.2) (layer "F.Cu") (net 2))
 (segment (start 145.735 91.765) (end 145.735 91.6) (width 0.2) (layer "F.Cu") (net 2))
 (segment (start 146.375 91.6) (end 146.826 92.051) (width 0.2) (layer "F.Cu") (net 40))
 (segment (start 146.826 92.051) (end 146.826 95.37504) (width 0.2) (layer "F.Cu") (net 40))
 (segment (start 146.826 95.37504) (end 146.70104 95.5) (width 0.2) (layer "F.Cu") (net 40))
 (segment (start 146.70104 95.5) (end 146.1 95.5) (width 0.2) (layer "F.Cu") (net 40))
 (segment (start 146.5 104.824999) (end 147.675001 106) (width 0.2) (layer "F.Cu") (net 6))
 (segment (start 150 105.9329) (end 150 105) (width 0.2) (layer "F.Cu") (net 6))
 (segment (start 146.5 103.85) (end 146.5 104.824999) (width 0.2) (layer "F.Cu") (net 6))
 (segment (start 150.5 104.5) (end 164.949 104.5) (width 0.2) (layer "F.Cu") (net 6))
 (segment (start 150 105) (end 150.5 104.5) (width 0.2) (layer "F.Cu") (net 6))
 (segment (start 147.675001 106) (end 149.9329 106) (width 0.2) (layer "F.Cu") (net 6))
 (segment (start 165.05 94.84) (end 166 94.84) (width 0.2) (layer "F.Cu") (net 6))
 (segment (start 149.9329 106) (end 150 105.9329) (width 0.2) (layer "F.Cu") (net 6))
 (segment (start 164.949 104.5) (end 164.949 94.941) (width 0.2) (layer "F.Cu") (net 6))
 (segment (start 164.949 94.941) (end 165.05 94.84) (width 0.2) (layer "F.Cu") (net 6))
 (segment (start 148.5 89.76) (end 147.968 89.76) (width 0.2) (layer "F.Cu") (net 5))
 (segment (start 145.23 102.875001) (end 145.23 103.85) (width 0.2) (layer "F.Cu") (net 5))
 (segment (start 147.449 90.279) (end 147.449 100.656001) (width 0.2) (layer "F.Cu") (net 5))
 (segment (start 147.968 89.76) (end 147.449 90.279) (width 0.2) (layer "F.Cu") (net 5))
 (segment (start 147.449 100.656001) (end 145.23 102.875001) (width 0.2) (layer "F.Cu") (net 5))
 (segment (start 150.5 105.5) (end 151 105) (width 0.2) (layer "F.Cu") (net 4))
 (segment (start 167.051 105.751) (end 167.051 91.551) (width 0.2) (layer "F.Cu") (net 4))
 (segment (start 166.53 91.03) (end 166 91.03) (width 0.2) (layer "F.Cu") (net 4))
 (segment (start 151 105) (end 164.949 105) (width 0.2) (layer "F.Cu") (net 4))
 (segment (start 142.69 104.824999) (end 144.365001 106.5) (width 0.2) (layer "F.Cu") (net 4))
 (segment (start 142.69 103.85) (end 142.69 104.824999) (width 0.2) (layer "F.Cu") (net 4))
 (segment (start 144.365001 106.5) (end 150.5 106.5) (width 0.2) (layer "F.Cu") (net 4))
 (segment (start 166.532 91.03) (end 166 91.03) (width 0.2) (layer "F.Cu") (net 4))
 (segment (start 164.949 105) (end 164.949 105.751) (width 0.2) (layer "F.Cu") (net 4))
 (segment (start 164.949 105.751) (end 167.051 105.751) (width 0.2) (layer "F.Cu") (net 4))
 (segment (start 150.5 106.5) (end 150.5 105.5) (width 0.2) (layer "F.Cu") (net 4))
 (segment (start 167.051 91.551) (end 166.53 91.03) (width 0.2) (layer "F.Cu") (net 4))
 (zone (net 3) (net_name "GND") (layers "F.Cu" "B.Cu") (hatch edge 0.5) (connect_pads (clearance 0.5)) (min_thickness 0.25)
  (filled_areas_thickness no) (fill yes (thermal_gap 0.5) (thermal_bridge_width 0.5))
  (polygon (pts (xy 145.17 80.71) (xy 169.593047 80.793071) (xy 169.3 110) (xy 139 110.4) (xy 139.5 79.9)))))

